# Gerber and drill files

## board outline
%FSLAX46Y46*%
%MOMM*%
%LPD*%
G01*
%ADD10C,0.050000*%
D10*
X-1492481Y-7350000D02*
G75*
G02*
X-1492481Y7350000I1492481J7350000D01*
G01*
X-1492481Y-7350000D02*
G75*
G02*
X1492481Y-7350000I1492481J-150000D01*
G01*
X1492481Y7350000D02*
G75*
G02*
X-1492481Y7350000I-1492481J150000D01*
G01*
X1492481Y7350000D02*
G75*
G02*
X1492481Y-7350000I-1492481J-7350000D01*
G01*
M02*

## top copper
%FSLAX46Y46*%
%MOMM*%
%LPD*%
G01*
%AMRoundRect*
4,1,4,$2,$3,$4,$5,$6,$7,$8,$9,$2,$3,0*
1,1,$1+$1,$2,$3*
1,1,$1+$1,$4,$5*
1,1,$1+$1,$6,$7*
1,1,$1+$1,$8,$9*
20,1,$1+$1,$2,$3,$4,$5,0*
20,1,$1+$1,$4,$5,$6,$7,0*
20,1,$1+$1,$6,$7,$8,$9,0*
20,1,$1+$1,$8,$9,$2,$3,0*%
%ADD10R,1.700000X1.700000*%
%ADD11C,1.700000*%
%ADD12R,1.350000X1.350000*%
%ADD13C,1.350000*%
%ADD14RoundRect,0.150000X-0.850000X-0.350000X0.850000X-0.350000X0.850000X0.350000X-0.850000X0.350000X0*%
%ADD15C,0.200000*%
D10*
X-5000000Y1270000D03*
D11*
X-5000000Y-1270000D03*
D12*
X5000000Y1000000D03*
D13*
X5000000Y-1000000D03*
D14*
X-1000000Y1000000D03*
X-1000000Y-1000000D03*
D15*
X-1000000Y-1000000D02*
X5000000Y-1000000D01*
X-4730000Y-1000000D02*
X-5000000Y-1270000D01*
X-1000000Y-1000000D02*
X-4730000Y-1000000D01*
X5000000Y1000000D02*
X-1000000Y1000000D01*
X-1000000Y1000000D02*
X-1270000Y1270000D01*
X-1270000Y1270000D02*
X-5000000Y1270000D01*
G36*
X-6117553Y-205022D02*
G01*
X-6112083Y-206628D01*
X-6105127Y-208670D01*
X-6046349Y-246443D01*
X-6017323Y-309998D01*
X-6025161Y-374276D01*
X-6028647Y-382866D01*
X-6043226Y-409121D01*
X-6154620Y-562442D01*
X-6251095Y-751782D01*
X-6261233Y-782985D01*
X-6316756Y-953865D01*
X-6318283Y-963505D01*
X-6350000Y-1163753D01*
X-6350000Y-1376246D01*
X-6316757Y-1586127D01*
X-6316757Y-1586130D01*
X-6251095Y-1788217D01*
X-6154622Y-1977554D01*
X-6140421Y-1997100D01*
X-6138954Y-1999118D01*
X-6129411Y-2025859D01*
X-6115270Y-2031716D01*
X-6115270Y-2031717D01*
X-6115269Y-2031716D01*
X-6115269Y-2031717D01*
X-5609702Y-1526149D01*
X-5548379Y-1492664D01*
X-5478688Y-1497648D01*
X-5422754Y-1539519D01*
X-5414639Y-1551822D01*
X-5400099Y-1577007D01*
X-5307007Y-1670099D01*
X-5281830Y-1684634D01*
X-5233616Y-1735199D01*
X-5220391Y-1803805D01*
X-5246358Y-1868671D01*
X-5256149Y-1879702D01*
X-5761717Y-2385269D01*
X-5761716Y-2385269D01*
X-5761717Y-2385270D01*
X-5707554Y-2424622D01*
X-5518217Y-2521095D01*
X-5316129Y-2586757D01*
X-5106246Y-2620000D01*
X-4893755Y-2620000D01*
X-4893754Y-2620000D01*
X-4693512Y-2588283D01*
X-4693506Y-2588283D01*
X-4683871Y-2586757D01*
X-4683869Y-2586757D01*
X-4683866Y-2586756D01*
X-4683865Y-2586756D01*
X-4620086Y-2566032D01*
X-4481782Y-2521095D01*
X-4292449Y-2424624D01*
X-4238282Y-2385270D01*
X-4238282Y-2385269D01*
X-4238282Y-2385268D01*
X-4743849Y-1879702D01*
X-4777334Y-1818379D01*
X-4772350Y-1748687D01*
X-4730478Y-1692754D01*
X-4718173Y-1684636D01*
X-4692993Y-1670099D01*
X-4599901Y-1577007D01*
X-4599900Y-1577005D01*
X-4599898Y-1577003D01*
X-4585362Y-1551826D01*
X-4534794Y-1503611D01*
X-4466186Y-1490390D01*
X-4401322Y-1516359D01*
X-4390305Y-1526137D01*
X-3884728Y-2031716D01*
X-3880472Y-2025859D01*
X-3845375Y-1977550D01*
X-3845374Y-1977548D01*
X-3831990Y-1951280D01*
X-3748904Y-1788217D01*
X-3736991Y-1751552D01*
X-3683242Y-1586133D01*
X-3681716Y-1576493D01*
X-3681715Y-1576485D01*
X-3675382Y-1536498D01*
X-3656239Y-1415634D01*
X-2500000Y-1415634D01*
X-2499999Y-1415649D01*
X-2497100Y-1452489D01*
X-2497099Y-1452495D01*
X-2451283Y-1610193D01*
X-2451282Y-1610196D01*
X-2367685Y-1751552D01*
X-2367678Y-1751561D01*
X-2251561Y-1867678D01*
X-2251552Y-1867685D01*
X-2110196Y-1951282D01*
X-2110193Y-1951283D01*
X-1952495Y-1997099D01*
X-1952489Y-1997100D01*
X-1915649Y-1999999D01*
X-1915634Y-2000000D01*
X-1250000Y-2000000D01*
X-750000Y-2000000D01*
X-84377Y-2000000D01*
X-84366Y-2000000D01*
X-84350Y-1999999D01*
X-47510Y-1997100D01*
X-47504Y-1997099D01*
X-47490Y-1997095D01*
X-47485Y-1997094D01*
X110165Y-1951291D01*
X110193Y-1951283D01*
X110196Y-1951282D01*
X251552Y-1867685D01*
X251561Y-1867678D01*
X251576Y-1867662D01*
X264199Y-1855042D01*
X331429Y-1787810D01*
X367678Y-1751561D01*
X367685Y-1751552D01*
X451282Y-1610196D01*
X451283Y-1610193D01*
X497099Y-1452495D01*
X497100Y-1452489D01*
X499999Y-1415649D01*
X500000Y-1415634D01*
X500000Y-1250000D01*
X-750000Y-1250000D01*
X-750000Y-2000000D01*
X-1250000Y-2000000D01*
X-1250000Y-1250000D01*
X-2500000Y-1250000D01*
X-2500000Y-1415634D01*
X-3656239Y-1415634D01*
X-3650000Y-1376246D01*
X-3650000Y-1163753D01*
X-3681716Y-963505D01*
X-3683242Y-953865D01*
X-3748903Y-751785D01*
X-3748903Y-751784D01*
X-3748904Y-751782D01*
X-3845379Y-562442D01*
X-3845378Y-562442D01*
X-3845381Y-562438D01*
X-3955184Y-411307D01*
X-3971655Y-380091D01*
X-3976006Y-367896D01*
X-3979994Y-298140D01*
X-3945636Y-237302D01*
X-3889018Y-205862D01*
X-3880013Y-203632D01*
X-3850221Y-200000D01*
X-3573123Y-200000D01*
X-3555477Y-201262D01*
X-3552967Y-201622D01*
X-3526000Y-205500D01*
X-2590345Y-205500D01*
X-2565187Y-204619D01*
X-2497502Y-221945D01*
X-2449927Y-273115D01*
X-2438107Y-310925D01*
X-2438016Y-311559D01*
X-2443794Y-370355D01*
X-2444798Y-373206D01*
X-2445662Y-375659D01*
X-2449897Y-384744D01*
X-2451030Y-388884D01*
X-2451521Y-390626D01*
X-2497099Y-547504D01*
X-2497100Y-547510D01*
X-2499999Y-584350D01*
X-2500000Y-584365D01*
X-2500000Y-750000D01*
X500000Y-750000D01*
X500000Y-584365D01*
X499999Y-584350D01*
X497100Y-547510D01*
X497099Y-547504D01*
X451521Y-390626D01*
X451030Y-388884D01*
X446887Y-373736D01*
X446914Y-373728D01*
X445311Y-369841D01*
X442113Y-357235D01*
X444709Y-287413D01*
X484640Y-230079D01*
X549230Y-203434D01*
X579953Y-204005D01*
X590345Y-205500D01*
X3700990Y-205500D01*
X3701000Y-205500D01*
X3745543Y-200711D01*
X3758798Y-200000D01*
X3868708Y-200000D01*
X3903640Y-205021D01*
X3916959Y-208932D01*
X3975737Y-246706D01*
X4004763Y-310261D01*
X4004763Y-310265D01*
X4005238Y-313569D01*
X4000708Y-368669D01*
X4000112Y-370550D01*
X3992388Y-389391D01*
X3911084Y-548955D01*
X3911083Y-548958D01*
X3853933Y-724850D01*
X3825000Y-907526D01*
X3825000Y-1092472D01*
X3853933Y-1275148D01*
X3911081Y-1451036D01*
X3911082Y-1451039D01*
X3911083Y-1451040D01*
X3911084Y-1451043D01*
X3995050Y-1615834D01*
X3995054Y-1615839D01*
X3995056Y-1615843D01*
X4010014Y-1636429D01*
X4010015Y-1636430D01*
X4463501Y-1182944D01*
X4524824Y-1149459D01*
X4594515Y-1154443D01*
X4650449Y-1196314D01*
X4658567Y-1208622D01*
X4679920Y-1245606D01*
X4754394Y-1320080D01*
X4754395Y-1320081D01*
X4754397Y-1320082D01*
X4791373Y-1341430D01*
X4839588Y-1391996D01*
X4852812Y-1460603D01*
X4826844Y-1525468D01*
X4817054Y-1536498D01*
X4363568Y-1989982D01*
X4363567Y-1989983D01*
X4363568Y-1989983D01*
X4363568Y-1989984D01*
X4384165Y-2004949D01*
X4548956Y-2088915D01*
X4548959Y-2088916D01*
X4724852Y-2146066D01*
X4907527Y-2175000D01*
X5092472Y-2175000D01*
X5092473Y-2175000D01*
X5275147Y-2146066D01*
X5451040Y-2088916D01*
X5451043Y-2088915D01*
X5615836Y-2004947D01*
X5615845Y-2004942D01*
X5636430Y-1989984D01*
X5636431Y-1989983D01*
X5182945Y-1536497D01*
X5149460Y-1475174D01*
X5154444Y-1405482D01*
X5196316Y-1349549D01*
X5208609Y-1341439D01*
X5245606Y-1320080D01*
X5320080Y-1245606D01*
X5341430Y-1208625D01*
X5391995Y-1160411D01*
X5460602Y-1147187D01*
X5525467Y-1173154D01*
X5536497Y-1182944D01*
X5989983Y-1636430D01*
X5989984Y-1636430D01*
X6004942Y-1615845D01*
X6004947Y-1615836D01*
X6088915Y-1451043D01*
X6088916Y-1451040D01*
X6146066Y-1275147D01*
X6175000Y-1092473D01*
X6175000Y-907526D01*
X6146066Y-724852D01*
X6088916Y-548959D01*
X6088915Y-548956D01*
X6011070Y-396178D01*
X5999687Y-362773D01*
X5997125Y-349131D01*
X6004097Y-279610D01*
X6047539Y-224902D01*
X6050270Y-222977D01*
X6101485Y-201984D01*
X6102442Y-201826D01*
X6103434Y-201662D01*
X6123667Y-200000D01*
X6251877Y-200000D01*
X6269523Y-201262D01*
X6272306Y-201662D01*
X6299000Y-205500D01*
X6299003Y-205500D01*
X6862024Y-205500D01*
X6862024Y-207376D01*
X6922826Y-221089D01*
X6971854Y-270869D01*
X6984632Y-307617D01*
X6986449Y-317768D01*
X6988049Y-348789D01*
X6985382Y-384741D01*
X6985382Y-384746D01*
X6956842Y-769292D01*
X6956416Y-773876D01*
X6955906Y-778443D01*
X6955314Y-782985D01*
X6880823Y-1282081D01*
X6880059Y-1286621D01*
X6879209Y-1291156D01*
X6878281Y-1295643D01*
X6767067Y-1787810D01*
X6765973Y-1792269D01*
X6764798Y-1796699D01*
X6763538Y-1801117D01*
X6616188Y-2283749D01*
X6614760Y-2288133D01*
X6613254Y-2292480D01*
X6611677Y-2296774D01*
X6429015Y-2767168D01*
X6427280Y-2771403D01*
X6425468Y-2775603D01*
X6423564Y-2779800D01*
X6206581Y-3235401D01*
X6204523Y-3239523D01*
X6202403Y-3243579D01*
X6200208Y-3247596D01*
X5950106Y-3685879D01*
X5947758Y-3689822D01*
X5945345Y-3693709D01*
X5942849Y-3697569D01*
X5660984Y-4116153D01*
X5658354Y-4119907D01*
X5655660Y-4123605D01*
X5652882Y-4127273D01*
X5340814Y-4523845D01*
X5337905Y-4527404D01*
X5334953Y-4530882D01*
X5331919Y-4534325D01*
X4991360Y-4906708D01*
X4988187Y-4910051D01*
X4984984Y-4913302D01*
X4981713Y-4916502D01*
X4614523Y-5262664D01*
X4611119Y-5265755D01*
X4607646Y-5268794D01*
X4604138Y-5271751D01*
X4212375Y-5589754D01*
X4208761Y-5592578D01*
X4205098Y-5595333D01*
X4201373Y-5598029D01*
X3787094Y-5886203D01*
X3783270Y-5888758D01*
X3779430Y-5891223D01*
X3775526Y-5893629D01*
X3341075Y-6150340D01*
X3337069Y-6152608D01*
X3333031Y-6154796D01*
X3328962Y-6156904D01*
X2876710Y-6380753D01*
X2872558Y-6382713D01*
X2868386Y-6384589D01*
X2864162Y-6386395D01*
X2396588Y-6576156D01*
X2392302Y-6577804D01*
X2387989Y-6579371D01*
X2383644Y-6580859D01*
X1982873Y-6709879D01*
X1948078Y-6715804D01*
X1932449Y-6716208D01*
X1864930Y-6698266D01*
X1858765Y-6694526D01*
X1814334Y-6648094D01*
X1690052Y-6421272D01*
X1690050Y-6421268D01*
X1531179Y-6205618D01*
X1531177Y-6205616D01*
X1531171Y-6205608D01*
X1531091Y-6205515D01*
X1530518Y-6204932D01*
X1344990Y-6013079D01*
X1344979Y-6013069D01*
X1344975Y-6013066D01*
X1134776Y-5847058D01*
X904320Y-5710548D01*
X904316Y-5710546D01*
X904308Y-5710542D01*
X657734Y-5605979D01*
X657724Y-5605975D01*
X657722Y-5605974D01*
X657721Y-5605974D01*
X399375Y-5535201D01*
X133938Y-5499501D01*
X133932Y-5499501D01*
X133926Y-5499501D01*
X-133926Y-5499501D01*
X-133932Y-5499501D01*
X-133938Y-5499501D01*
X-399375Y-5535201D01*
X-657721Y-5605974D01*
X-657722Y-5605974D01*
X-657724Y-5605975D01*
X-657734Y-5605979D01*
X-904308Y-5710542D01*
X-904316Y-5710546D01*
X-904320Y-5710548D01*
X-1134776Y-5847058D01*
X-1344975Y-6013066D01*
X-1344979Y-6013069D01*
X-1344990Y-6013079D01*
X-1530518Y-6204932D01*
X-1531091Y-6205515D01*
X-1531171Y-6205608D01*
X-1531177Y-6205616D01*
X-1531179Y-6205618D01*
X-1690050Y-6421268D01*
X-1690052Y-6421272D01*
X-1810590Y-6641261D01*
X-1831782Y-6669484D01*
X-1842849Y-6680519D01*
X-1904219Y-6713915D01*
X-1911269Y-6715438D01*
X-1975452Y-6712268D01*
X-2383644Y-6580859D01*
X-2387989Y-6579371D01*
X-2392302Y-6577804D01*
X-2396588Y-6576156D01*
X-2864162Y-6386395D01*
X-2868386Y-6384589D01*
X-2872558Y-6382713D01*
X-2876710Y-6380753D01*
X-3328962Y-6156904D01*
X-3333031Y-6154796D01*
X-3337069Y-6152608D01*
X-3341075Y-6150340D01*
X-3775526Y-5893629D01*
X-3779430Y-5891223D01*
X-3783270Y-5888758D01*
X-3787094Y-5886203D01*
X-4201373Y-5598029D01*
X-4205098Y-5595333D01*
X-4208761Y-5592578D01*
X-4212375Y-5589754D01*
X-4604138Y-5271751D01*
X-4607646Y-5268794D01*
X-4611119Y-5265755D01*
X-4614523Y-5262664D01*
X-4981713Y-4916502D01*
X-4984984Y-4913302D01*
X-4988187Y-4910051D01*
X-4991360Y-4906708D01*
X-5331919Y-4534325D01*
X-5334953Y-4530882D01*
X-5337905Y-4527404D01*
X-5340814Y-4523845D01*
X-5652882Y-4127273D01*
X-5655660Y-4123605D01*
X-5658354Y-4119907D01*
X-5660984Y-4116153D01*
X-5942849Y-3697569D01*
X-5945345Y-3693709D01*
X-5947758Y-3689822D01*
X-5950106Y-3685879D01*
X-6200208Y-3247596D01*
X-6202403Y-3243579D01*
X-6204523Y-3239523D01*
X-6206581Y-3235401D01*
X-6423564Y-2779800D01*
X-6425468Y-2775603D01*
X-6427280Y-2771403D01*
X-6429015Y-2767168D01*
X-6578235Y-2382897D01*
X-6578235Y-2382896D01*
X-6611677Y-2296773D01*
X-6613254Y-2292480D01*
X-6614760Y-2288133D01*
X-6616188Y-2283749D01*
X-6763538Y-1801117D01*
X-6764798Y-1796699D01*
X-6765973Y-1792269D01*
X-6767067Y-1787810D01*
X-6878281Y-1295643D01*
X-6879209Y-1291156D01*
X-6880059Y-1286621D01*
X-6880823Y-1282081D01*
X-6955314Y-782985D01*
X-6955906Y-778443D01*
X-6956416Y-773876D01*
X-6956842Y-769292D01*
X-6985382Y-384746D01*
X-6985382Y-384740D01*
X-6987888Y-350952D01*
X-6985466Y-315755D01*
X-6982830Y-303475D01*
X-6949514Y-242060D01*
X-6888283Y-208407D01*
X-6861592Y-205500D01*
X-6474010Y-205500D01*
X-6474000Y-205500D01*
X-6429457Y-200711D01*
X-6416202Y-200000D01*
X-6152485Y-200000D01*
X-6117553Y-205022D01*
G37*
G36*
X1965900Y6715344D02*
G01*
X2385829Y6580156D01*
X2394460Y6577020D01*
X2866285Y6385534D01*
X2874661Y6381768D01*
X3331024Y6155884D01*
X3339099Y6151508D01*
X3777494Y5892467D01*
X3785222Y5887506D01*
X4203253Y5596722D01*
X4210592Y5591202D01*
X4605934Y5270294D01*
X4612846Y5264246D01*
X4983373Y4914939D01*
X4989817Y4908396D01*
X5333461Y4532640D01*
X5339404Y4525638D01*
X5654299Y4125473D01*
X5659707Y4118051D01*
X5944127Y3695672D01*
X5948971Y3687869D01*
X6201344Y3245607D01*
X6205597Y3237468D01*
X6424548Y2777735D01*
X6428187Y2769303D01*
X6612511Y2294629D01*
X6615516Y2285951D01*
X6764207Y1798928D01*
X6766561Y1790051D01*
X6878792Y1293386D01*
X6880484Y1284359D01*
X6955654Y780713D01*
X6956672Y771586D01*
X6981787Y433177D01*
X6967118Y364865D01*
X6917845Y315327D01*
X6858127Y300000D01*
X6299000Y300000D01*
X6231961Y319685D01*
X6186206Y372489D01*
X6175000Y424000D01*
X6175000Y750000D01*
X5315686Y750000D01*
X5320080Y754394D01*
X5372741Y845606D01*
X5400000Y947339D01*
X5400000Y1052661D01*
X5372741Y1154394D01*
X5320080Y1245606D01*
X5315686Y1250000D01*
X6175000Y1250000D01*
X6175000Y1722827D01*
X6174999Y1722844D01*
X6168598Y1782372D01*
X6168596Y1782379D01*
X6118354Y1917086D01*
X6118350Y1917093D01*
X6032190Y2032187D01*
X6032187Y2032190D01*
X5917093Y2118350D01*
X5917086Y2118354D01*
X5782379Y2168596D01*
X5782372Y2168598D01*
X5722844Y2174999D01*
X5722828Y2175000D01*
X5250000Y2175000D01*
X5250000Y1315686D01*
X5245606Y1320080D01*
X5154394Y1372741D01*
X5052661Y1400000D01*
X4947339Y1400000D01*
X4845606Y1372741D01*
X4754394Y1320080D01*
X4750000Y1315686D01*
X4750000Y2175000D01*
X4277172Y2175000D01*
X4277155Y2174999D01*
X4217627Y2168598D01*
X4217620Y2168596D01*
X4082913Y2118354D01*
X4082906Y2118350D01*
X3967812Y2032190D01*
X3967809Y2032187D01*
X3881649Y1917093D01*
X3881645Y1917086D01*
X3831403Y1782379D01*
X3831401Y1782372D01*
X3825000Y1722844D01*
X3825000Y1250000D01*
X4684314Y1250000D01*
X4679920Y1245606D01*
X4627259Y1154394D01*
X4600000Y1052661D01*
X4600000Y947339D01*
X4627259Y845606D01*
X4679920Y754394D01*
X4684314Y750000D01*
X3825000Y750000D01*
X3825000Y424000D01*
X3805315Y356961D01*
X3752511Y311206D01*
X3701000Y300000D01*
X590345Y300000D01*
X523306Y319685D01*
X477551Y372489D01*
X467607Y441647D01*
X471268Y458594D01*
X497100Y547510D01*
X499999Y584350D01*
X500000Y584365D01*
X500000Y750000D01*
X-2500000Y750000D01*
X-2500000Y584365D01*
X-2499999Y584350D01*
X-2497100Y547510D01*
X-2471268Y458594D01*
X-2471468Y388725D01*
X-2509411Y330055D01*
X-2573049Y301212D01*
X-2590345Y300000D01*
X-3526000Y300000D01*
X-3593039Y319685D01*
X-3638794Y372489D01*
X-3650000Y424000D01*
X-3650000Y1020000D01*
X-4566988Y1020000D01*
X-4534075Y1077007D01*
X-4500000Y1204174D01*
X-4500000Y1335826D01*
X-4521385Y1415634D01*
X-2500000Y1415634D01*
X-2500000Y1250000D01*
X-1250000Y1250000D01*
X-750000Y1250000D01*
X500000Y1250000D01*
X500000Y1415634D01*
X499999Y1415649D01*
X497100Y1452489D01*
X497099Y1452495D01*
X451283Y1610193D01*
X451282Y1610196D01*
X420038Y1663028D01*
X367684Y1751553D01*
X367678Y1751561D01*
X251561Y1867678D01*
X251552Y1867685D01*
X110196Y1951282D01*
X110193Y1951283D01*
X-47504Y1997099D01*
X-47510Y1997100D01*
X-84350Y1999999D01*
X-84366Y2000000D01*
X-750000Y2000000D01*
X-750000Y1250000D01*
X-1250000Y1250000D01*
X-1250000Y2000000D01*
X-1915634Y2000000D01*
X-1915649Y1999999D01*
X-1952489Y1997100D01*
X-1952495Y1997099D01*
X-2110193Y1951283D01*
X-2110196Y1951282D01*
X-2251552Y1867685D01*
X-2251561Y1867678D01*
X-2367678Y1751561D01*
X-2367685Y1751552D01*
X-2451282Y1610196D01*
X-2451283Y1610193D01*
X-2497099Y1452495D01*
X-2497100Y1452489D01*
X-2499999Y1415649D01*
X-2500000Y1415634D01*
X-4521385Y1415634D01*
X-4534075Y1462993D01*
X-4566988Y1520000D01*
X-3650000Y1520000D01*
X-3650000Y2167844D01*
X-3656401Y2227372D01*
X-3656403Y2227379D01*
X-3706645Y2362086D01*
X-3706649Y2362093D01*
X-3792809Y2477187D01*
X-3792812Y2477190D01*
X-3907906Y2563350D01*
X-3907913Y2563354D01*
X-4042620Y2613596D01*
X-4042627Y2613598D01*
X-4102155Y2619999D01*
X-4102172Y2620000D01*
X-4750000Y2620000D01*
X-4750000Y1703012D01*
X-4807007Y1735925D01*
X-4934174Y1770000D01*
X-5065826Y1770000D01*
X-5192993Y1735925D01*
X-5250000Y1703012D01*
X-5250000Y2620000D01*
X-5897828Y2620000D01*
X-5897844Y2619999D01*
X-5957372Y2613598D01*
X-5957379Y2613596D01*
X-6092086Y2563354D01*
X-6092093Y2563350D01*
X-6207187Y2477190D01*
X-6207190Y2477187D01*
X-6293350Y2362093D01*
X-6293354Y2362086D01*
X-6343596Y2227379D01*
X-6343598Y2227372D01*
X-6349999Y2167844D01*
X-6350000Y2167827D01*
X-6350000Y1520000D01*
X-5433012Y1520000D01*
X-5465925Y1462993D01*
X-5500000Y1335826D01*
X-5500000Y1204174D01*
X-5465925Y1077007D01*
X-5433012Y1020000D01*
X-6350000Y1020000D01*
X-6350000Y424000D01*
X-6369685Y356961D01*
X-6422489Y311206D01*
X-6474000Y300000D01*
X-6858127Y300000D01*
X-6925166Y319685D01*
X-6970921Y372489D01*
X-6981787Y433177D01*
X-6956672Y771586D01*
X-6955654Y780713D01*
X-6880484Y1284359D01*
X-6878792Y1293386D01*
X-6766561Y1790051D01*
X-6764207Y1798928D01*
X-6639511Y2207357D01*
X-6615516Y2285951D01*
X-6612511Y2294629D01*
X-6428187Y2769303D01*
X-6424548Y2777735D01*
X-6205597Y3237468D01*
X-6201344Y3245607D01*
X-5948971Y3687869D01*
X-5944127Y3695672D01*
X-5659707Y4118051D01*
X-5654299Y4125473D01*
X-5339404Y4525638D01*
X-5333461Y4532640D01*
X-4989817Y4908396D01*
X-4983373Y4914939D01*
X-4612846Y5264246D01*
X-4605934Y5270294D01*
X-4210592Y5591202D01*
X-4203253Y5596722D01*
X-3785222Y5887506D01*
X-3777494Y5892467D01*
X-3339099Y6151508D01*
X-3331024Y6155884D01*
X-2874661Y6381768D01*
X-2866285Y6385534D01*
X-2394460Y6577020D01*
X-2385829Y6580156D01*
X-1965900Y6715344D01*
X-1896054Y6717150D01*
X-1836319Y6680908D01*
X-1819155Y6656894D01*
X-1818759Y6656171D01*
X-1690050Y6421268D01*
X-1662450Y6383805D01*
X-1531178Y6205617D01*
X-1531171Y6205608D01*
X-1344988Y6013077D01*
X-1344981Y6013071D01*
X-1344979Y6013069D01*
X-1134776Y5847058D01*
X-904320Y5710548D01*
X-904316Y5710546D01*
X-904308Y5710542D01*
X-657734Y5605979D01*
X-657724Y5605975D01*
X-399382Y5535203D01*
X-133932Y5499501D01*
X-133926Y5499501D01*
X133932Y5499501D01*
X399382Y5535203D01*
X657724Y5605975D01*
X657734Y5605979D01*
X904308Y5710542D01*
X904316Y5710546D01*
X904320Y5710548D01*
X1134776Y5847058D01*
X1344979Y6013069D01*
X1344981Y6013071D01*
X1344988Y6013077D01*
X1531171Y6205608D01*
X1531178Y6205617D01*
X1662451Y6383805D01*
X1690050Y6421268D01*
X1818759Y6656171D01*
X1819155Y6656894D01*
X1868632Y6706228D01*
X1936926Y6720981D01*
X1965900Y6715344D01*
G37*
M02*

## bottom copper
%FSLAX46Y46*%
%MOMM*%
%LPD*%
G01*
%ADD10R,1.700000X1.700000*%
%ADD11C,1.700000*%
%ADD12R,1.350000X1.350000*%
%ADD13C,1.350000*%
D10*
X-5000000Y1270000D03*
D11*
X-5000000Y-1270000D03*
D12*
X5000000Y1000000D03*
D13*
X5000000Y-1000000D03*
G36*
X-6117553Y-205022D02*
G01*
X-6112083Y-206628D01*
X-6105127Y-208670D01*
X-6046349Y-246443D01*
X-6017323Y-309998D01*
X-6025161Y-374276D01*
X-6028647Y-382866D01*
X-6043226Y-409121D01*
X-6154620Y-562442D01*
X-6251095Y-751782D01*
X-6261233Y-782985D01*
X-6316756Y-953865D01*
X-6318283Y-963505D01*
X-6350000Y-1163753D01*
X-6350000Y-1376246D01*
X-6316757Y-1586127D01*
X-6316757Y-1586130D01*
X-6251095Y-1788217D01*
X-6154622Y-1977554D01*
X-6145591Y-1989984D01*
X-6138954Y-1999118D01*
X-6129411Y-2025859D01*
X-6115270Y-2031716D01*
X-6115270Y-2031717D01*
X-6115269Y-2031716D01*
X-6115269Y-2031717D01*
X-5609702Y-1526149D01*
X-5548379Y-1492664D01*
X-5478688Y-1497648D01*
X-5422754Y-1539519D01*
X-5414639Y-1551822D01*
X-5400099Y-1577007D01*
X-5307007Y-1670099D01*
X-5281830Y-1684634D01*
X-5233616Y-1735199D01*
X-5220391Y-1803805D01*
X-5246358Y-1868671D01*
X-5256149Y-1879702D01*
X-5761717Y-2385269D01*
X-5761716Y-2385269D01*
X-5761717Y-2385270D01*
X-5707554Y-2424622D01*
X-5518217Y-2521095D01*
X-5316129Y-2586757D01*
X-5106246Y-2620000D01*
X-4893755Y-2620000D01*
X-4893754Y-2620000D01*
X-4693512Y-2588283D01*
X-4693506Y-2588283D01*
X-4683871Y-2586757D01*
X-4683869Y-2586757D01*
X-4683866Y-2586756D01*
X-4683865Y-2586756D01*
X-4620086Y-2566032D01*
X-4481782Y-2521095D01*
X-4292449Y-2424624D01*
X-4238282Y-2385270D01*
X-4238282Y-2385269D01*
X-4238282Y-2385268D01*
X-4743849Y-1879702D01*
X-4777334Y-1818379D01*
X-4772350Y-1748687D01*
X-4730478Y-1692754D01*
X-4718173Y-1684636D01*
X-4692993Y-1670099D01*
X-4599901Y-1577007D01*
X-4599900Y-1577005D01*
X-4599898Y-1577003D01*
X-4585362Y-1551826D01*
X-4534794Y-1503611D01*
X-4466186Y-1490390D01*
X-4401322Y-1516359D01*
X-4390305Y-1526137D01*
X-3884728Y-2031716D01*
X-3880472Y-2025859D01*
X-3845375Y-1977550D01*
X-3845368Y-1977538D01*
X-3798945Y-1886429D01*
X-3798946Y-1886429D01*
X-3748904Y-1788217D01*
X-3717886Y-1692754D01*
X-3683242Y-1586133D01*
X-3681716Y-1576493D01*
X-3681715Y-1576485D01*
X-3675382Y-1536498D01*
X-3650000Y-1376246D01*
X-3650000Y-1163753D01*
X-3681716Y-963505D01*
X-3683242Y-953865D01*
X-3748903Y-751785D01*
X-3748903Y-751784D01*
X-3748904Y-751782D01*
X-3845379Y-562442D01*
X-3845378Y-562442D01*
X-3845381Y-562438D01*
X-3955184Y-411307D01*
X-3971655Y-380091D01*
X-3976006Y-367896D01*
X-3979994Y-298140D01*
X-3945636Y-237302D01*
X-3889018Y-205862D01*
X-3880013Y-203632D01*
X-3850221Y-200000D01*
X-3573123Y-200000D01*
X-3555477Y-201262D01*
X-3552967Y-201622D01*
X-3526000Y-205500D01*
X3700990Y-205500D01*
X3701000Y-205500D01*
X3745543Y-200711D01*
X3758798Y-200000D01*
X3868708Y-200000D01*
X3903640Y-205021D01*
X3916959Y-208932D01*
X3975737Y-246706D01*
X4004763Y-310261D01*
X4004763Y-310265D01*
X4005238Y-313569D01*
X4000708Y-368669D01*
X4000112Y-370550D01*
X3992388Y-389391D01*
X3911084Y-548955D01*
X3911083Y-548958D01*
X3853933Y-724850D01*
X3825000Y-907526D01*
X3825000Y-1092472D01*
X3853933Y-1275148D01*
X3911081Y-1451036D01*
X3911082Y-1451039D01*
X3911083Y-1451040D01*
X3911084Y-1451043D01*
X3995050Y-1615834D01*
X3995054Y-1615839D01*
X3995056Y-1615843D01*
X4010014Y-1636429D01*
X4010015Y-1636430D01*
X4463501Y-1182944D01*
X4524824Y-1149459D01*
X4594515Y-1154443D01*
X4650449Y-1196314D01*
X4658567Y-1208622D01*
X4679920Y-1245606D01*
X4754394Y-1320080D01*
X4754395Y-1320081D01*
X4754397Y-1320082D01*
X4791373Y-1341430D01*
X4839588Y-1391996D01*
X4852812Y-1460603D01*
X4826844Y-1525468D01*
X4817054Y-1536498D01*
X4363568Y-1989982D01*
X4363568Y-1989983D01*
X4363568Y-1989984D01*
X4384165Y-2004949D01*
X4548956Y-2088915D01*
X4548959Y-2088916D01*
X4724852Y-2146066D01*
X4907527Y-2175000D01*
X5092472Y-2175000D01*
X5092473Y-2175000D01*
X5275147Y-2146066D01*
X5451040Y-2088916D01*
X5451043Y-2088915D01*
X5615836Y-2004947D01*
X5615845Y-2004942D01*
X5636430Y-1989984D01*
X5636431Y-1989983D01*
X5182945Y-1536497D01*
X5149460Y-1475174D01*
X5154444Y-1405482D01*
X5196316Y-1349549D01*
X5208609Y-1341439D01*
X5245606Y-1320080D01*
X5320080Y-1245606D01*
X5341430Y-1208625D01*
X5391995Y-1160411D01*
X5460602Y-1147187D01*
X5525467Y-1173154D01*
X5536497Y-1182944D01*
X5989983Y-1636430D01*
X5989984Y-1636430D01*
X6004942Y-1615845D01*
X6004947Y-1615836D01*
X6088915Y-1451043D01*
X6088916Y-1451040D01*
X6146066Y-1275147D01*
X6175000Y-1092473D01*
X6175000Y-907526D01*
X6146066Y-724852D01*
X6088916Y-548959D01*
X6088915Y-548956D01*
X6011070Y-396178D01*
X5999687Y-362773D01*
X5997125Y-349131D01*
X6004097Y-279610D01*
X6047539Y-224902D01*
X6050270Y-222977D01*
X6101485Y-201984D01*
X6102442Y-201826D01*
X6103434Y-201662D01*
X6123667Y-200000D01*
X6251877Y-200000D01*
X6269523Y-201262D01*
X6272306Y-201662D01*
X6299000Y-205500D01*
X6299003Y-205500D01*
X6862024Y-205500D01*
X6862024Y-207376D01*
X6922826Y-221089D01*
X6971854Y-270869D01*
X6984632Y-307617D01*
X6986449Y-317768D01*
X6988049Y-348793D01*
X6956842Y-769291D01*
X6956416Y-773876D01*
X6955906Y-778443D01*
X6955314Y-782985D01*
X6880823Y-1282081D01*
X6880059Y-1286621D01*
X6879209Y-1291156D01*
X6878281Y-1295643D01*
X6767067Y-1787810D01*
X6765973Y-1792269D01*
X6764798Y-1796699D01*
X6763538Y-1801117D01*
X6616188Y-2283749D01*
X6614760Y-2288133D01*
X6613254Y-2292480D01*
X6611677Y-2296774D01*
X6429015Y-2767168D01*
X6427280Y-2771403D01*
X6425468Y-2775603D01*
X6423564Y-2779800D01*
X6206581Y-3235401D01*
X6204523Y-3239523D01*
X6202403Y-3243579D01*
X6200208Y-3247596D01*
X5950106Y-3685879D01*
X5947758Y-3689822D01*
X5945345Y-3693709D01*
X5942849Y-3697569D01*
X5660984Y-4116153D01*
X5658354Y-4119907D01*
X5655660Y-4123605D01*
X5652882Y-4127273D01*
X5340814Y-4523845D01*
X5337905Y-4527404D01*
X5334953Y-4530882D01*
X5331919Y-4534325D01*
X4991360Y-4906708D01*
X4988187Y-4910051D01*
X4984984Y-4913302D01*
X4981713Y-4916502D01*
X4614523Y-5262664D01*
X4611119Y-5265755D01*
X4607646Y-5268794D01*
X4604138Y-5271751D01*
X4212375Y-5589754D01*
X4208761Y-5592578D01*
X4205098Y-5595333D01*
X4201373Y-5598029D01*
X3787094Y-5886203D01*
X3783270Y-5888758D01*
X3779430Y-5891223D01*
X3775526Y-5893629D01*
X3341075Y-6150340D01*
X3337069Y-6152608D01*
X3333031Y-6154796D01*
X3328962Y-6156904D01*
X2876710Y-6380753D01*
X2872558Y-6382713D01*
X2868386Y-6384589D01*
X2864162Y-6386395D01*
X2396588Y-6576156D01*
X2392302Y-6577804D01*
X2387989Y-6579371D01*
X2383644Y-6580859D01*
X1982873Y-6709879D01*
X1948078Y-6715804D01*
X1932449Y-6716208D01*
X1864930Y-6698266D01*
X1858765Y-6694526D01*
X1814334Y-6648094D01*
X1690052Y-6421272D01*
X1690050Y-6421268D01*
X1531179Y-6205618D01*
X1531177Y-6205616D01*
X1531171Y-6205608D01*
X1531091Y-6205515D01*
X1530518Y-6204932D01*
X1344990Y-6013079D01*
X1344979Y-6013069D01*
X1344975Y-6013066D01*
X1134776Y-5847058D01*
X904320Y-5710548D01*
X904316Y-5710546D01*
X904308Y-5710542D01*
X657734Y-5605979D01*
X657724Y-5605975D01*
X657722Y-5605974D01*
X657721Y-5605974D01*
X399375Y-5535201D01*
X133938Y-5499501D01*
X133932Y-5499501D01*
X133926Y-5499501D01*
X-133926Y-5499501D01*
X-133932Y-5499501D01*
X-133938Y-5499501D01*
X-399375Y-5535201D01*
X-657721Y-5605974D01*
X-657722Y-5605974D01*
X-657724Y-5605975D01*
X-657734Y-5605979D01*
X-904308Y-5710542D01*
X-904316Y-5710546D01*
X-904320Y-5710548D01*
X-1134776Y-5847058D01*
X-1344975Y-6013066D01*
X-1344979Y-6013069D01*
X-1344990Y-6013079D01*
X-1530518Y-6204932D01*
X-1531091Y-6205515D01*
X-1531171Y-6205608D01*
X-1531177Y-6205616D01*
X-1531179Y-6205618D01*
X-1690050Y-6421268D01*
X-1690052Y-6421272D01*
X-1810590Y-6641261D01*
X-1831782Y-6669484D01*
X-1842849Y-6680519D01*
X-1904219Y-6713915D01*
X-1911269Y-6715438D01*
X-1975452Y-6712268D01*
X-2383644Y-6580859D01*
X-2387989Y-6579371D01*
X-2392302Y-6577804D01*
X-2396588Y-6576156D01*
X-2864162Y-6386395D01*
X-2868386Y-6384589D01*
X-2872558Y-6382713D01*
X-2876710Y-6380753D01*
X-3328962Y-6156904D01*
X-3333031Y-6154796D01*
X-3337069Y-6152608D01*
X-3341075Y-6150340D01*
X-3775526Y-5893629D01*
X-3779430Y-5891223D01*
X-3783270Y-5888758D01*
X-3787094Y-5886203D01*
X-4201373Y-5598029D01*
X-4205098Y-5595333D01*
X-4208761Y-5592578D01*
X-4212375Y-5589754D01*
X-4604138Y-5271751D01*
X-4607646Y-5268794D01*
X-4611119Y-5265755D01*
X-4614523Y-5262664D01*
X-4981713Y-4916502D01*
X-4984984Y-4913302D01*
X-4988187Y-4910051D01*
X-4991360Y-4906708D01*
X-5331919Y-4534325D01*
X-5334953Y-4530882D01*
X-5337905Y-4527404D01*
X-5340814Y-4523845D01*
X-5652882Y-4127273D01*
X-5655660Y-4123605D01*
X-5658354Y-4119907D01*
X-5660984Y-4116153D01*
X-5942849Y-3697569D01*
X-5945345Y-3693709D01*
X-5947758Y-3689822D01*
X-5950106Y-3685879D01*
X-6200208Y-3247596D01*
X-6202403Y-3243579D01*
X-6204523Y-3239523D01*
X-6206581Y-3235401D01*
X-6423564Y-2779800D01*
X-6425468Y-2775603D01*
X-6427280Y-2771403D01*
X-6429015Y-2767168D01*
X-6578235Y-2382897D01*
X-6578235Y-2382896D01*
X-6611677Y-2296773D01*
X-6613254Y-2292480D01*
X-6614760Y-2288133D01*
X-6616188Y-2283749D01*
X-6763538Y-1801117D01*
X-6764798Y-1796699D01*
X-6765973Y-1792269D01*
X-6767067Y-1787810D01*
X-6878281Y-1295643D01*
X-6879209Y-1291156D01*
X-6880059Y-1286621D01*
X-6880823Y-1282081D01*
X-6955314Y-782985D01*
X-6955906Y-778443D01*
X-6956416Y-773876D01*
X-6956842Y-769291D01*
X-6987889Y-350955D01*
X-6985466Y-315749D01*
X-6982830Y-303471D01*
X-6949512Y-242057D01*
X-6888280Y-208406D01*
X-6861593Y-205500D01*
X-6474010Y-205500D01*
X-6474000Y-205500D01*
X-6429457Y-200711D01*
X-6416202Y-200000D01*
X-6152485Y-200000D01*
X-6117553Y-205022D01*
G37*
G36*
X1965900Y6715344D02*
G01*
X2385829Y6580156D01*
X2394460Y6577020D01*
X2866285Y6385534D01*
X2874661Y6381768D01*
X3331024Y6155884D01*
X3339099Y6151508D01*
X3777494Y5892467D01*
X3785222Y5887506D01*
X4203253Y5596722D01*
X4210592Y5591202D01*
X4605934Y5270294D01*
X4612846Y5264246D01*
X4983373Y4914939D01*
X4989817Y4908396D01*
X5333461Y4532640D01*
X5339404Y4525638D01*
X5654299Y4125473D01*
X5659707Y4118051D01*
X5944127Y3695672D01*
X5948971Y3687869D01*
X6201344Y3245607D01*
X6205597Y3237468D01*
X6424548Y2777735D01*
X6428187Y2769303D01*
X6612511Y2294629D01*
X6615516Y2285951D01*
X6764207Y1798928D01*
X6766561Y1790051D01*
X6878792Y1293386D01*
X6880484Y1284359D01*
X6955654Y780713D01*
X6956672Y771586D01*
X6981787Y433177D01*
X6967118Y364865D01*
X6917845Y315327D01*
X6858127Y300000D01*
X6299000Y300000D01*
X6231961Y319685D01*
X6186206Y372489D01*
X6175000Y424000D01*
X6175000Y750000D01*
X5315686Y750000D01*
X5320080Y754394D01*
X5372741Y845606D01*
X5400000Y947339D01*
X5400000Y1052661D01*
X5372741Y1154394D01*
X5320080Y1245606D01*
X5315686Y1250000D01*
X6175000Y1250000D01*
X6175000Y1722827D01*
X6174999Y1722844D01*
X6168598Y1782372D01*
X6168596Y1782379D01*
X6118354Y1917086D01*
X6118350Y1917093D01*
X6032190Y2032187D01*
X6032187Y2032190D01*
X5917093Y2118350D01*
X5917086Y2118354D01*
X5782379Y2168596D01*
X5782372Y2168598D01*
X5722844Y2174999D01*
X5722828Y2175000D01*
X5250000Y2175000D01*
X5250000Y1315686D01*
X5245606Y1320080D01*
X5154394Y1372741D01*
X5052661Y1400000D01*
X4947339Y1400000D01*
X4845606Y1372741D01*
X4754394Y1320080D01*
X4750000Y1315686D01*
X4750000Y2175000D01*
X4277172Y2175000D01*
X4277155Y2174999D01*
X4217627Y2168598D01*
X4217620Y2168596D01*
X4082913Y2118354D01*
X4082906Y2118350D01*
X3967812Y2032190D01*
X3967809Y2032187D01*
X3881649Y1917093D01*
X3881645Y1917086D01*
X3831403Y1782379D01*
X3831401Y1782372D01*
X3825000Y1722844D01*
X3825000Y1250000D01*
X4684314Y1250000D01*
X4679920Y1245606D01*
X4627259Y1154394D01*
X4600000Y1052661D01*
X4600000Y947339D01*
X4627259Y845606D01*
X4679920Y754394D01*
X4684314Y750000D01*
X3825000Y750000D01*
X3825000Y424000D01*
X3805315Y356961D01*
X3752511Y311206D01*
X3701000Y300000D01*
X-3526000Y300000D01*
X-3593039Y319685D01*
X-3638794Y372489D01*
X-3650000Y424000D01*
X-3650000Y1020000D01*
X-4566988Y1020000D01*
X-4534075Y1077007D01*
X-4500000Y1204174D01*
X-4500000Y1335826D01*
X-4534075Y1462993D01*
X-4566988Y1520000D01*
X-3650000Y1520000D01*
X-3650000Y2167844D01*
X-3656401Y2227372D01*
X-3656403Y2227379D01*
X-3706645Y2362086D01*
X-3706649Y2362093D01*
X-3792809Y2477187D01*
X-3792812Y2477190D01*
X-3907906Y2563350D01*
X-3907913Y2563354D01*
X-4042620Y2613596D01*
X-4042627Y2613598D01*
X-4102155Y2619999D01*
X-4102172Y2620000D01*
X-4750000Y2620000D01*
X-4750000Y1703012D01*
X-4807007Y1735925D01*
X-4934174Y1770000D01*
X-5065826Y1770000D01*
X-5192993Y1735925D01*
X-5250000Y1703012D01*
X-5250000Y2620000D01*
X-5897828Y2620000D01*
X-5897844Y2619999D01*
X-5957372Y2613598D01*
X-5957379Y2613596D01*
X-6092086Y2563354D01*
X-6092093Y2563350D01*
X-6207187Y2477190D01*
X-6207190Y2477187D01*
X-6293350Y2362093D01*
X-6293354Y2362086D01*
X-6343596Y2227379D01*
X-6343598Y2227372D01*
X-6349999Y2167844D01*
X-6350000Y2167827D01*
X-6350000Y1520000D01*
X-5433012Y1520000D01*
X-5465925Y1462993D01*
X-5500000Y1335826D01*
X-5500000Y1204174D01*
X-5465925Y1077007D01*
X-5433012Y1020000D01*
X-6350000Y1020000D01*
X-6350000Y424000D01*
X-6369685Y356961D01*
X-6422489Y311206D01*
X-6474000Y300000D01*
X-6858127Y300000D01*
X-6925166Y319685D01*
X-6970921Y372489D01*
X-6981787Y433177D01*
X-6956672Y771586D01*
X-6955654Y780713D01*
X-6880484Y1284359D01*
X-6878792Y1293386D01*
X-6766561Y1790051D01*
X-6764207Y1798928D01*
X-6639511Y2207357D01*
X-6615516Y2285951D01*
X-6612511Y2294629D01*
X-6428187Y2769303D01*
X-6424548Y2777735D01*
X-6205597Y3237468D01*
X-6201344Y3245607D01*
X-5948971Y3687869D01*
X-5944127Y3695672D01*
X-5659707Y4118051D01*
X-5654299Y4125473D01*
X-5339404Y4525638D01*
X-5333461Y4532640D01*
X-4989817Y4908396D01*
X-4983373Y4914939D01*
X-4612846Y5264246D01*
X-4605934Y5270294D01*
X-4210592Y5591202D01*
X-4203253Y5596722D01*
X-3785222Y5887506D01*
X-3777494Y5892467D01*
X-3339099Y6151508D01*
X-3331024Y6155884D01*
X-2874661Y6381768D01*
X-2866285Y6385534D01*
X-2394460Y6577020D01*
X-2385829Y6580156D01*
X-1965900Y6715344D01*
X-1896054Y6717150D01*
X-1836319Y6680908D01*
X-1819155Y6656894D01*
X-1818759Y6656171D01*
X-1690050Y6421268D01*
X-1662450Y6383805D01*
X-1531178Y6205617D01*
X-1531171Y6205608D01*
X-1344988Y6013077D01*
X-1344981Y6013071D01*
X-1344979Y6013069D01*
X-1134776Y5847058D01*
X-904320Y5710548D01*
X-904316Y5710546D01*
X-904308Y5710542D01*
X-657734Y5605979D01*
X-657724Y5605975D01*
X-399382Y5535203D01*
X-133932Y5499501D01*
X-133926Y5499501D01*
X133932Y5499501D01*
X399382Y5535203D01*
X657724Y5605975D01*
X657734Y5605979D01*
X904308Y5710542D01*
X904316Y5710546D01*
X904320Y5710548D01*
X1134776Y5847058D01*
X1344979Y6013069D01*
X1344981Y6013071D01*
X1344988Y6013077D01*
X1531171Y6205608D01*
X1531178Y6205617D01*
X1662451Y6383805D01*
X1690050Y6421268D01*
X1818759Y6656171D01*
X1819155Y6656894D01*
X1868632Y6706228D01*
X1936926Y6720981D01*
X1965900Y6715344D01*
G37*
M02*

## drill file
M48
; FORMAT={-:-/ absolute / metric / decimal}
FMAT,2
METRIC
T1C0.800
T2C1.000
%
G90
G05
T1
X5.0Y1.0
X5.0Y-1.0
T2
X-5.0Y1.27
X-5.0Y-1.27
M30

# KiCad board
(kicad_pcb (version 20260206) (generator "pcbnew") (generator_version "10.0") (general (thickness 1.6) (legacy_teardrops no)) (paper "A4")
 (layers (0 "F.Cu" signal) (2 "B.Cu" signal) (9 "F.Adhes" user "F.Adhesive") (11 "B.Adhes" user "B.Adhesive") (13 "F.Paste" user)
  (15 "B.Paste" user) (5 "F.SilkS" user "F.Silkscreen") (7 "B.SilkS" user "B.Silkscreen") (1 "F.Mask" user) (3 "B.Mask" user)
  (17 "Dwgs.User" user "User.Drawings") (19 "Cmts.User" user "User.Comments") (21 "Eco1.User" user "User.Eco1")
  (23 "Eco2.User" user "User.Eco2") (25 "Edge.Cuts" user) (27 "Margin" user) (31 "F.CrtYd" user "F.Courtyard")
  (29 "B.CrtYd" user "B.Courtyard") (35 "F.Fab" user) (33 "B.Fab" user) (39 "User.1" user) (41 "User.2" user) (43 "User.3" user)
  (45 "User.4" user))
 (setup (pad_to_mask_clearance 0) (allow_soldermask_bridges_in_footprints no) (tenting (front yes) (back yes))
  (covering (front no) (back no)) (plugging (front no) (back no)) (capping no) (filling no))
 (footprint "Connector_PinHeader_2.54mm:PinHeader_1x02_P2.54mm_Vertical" (layer "F.Cu") (at -5 -1.27)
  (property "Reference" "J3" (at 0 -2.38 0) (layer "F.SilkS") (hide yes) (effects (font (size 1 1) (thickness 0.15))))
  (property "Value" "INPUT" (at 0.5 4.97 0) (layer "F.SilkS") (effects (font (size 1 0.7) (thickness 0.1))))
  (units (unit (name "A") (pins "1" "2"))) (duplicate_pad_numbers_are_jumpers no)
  (pad "1" thru_hole rect (at 0 0) (size 1.7 1.7) (drill 1) (layers "*.Cu" "*.Mask") (remove_unused_layers no) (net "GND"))
  (pad "2" thru_hole circle (at 0 2.54) (size 1.7 1.7) (drill 1) (layers "*.Cu" "*.Mask") (remove_unused_layers no) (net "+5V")))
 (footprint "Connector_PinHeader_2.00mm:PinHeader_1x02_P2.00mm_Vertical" (layer "F.Cu") (at 5 -1)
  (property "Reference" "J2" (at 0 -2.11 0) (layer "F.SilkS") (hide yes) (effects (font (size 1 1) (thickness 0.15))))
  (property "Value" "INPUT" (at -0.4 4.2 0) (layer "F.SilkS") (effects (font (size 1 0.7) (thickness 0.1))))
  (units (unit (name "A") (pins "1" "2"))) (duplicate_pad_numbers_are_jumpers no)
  (pad "1" thru_hole rect (at 0 0) (size 1.35 1.35) (drill 0.8) (layers "*.Cu" "*.Mask") (remove_unused_layers no) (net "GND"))
  (pad "2" thru_hole circle (at 0 2) (size 1.35 1.35) (drill 0.8) (layers "*.Cu" "*.Mask") (remove_unused_layers no) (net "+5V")))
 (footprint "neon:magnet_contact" (layer "F.Cu") (at 0 0 -90)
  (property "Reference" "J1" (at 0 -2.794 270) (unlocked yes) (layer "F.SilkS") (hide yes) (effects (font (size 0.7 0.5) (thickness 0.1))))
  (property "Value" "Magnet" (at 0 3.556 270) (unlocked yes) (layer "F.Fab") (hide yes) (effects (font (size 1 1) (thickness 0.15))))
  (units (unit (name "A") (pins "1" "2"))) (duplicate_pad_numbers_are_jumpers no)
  (pad "1" smd roundrect (at -1 1) (size 2 1) (layers "F.Cu" "F.Mask" "F.Paste") (roundrect_rratio 0.15) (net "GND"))
  (pad "2" smd roundrect (at 1 1) (size 2 1) (layers "F.Cu" "F.Mask" "F.Paste") (roundrect_rratio 0.15) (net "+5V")))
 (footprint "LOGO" (layer "B.Cu") (at 0 0 -90)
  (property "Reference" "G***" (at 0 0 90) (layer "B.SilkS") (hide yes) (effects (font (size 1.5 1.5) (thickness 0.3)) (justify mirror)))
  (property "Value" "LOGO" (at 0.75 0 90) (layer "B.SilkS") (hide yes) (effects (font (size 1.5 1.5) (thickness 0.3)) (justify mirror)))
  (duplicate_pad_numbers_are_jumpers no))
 (gr_arc (start -1.492481 7.35) (mid -7.5 0) (end -1.492481 -7.35) (stroke (width 0.05) (type default)) (layer "Edge.Cuts"))
 (gr_arc (start -1.492481 7.35) (mid 0 6) (end 1.492481 7.35) (stroke (width 0.05) (type default)) (layer "Edge.Cuts"))
 (gr_arc (start 1.492481 -7.35) (mid 0 -6) (end -1.492481 -7.35) (stroke (width 0.05) (type default)) (layer "Edge.Cuts"))
 (gr_arc (start 1.492481 -7.35) (mid 7.5 0) (end 1.492481 7.35) (stroke (width 0.05) (type default)) (layer "Edge.Cuts"))
 (segment (start -1 1) (end 5 1) (width 0.2) (layer "F.Cu") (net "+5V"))
 (segment (start -4.73 1) (end -5 1.27) (width 0.2) (layer "F.Cu") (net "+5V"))
 (segment (start -1 1) (end -4.73 1) (width 0.2) (layer "F.Cu") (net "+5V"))
 (segment (start 5 -1) (end -1 -1) (width 0.2) (layer "F.Cu") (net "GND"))
 (segment (start -1 -1) (end -1.27 -1.27) (width 0.2) (layer "F.Cu") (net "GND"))
 (segment (start -1.27 -1.27) (end -5 -1.27) (width 0.2) (layer "F.Cu") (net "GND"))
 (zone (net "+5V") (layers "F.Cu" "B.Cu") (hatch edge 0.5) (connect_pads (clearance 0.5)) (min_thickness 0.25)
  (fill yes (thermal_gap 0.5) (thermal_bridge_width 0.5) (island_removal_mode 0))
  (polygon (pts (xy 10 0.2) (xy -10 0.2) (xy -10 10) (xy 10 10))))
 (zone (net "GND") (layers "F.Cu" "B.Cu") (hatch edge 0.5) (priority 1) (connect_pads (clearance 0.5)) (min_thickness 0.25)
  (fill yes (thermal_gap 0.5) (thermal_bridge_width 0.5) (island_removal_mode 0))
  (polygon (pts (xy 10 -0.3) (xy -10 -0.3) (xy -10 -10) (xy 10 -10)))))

